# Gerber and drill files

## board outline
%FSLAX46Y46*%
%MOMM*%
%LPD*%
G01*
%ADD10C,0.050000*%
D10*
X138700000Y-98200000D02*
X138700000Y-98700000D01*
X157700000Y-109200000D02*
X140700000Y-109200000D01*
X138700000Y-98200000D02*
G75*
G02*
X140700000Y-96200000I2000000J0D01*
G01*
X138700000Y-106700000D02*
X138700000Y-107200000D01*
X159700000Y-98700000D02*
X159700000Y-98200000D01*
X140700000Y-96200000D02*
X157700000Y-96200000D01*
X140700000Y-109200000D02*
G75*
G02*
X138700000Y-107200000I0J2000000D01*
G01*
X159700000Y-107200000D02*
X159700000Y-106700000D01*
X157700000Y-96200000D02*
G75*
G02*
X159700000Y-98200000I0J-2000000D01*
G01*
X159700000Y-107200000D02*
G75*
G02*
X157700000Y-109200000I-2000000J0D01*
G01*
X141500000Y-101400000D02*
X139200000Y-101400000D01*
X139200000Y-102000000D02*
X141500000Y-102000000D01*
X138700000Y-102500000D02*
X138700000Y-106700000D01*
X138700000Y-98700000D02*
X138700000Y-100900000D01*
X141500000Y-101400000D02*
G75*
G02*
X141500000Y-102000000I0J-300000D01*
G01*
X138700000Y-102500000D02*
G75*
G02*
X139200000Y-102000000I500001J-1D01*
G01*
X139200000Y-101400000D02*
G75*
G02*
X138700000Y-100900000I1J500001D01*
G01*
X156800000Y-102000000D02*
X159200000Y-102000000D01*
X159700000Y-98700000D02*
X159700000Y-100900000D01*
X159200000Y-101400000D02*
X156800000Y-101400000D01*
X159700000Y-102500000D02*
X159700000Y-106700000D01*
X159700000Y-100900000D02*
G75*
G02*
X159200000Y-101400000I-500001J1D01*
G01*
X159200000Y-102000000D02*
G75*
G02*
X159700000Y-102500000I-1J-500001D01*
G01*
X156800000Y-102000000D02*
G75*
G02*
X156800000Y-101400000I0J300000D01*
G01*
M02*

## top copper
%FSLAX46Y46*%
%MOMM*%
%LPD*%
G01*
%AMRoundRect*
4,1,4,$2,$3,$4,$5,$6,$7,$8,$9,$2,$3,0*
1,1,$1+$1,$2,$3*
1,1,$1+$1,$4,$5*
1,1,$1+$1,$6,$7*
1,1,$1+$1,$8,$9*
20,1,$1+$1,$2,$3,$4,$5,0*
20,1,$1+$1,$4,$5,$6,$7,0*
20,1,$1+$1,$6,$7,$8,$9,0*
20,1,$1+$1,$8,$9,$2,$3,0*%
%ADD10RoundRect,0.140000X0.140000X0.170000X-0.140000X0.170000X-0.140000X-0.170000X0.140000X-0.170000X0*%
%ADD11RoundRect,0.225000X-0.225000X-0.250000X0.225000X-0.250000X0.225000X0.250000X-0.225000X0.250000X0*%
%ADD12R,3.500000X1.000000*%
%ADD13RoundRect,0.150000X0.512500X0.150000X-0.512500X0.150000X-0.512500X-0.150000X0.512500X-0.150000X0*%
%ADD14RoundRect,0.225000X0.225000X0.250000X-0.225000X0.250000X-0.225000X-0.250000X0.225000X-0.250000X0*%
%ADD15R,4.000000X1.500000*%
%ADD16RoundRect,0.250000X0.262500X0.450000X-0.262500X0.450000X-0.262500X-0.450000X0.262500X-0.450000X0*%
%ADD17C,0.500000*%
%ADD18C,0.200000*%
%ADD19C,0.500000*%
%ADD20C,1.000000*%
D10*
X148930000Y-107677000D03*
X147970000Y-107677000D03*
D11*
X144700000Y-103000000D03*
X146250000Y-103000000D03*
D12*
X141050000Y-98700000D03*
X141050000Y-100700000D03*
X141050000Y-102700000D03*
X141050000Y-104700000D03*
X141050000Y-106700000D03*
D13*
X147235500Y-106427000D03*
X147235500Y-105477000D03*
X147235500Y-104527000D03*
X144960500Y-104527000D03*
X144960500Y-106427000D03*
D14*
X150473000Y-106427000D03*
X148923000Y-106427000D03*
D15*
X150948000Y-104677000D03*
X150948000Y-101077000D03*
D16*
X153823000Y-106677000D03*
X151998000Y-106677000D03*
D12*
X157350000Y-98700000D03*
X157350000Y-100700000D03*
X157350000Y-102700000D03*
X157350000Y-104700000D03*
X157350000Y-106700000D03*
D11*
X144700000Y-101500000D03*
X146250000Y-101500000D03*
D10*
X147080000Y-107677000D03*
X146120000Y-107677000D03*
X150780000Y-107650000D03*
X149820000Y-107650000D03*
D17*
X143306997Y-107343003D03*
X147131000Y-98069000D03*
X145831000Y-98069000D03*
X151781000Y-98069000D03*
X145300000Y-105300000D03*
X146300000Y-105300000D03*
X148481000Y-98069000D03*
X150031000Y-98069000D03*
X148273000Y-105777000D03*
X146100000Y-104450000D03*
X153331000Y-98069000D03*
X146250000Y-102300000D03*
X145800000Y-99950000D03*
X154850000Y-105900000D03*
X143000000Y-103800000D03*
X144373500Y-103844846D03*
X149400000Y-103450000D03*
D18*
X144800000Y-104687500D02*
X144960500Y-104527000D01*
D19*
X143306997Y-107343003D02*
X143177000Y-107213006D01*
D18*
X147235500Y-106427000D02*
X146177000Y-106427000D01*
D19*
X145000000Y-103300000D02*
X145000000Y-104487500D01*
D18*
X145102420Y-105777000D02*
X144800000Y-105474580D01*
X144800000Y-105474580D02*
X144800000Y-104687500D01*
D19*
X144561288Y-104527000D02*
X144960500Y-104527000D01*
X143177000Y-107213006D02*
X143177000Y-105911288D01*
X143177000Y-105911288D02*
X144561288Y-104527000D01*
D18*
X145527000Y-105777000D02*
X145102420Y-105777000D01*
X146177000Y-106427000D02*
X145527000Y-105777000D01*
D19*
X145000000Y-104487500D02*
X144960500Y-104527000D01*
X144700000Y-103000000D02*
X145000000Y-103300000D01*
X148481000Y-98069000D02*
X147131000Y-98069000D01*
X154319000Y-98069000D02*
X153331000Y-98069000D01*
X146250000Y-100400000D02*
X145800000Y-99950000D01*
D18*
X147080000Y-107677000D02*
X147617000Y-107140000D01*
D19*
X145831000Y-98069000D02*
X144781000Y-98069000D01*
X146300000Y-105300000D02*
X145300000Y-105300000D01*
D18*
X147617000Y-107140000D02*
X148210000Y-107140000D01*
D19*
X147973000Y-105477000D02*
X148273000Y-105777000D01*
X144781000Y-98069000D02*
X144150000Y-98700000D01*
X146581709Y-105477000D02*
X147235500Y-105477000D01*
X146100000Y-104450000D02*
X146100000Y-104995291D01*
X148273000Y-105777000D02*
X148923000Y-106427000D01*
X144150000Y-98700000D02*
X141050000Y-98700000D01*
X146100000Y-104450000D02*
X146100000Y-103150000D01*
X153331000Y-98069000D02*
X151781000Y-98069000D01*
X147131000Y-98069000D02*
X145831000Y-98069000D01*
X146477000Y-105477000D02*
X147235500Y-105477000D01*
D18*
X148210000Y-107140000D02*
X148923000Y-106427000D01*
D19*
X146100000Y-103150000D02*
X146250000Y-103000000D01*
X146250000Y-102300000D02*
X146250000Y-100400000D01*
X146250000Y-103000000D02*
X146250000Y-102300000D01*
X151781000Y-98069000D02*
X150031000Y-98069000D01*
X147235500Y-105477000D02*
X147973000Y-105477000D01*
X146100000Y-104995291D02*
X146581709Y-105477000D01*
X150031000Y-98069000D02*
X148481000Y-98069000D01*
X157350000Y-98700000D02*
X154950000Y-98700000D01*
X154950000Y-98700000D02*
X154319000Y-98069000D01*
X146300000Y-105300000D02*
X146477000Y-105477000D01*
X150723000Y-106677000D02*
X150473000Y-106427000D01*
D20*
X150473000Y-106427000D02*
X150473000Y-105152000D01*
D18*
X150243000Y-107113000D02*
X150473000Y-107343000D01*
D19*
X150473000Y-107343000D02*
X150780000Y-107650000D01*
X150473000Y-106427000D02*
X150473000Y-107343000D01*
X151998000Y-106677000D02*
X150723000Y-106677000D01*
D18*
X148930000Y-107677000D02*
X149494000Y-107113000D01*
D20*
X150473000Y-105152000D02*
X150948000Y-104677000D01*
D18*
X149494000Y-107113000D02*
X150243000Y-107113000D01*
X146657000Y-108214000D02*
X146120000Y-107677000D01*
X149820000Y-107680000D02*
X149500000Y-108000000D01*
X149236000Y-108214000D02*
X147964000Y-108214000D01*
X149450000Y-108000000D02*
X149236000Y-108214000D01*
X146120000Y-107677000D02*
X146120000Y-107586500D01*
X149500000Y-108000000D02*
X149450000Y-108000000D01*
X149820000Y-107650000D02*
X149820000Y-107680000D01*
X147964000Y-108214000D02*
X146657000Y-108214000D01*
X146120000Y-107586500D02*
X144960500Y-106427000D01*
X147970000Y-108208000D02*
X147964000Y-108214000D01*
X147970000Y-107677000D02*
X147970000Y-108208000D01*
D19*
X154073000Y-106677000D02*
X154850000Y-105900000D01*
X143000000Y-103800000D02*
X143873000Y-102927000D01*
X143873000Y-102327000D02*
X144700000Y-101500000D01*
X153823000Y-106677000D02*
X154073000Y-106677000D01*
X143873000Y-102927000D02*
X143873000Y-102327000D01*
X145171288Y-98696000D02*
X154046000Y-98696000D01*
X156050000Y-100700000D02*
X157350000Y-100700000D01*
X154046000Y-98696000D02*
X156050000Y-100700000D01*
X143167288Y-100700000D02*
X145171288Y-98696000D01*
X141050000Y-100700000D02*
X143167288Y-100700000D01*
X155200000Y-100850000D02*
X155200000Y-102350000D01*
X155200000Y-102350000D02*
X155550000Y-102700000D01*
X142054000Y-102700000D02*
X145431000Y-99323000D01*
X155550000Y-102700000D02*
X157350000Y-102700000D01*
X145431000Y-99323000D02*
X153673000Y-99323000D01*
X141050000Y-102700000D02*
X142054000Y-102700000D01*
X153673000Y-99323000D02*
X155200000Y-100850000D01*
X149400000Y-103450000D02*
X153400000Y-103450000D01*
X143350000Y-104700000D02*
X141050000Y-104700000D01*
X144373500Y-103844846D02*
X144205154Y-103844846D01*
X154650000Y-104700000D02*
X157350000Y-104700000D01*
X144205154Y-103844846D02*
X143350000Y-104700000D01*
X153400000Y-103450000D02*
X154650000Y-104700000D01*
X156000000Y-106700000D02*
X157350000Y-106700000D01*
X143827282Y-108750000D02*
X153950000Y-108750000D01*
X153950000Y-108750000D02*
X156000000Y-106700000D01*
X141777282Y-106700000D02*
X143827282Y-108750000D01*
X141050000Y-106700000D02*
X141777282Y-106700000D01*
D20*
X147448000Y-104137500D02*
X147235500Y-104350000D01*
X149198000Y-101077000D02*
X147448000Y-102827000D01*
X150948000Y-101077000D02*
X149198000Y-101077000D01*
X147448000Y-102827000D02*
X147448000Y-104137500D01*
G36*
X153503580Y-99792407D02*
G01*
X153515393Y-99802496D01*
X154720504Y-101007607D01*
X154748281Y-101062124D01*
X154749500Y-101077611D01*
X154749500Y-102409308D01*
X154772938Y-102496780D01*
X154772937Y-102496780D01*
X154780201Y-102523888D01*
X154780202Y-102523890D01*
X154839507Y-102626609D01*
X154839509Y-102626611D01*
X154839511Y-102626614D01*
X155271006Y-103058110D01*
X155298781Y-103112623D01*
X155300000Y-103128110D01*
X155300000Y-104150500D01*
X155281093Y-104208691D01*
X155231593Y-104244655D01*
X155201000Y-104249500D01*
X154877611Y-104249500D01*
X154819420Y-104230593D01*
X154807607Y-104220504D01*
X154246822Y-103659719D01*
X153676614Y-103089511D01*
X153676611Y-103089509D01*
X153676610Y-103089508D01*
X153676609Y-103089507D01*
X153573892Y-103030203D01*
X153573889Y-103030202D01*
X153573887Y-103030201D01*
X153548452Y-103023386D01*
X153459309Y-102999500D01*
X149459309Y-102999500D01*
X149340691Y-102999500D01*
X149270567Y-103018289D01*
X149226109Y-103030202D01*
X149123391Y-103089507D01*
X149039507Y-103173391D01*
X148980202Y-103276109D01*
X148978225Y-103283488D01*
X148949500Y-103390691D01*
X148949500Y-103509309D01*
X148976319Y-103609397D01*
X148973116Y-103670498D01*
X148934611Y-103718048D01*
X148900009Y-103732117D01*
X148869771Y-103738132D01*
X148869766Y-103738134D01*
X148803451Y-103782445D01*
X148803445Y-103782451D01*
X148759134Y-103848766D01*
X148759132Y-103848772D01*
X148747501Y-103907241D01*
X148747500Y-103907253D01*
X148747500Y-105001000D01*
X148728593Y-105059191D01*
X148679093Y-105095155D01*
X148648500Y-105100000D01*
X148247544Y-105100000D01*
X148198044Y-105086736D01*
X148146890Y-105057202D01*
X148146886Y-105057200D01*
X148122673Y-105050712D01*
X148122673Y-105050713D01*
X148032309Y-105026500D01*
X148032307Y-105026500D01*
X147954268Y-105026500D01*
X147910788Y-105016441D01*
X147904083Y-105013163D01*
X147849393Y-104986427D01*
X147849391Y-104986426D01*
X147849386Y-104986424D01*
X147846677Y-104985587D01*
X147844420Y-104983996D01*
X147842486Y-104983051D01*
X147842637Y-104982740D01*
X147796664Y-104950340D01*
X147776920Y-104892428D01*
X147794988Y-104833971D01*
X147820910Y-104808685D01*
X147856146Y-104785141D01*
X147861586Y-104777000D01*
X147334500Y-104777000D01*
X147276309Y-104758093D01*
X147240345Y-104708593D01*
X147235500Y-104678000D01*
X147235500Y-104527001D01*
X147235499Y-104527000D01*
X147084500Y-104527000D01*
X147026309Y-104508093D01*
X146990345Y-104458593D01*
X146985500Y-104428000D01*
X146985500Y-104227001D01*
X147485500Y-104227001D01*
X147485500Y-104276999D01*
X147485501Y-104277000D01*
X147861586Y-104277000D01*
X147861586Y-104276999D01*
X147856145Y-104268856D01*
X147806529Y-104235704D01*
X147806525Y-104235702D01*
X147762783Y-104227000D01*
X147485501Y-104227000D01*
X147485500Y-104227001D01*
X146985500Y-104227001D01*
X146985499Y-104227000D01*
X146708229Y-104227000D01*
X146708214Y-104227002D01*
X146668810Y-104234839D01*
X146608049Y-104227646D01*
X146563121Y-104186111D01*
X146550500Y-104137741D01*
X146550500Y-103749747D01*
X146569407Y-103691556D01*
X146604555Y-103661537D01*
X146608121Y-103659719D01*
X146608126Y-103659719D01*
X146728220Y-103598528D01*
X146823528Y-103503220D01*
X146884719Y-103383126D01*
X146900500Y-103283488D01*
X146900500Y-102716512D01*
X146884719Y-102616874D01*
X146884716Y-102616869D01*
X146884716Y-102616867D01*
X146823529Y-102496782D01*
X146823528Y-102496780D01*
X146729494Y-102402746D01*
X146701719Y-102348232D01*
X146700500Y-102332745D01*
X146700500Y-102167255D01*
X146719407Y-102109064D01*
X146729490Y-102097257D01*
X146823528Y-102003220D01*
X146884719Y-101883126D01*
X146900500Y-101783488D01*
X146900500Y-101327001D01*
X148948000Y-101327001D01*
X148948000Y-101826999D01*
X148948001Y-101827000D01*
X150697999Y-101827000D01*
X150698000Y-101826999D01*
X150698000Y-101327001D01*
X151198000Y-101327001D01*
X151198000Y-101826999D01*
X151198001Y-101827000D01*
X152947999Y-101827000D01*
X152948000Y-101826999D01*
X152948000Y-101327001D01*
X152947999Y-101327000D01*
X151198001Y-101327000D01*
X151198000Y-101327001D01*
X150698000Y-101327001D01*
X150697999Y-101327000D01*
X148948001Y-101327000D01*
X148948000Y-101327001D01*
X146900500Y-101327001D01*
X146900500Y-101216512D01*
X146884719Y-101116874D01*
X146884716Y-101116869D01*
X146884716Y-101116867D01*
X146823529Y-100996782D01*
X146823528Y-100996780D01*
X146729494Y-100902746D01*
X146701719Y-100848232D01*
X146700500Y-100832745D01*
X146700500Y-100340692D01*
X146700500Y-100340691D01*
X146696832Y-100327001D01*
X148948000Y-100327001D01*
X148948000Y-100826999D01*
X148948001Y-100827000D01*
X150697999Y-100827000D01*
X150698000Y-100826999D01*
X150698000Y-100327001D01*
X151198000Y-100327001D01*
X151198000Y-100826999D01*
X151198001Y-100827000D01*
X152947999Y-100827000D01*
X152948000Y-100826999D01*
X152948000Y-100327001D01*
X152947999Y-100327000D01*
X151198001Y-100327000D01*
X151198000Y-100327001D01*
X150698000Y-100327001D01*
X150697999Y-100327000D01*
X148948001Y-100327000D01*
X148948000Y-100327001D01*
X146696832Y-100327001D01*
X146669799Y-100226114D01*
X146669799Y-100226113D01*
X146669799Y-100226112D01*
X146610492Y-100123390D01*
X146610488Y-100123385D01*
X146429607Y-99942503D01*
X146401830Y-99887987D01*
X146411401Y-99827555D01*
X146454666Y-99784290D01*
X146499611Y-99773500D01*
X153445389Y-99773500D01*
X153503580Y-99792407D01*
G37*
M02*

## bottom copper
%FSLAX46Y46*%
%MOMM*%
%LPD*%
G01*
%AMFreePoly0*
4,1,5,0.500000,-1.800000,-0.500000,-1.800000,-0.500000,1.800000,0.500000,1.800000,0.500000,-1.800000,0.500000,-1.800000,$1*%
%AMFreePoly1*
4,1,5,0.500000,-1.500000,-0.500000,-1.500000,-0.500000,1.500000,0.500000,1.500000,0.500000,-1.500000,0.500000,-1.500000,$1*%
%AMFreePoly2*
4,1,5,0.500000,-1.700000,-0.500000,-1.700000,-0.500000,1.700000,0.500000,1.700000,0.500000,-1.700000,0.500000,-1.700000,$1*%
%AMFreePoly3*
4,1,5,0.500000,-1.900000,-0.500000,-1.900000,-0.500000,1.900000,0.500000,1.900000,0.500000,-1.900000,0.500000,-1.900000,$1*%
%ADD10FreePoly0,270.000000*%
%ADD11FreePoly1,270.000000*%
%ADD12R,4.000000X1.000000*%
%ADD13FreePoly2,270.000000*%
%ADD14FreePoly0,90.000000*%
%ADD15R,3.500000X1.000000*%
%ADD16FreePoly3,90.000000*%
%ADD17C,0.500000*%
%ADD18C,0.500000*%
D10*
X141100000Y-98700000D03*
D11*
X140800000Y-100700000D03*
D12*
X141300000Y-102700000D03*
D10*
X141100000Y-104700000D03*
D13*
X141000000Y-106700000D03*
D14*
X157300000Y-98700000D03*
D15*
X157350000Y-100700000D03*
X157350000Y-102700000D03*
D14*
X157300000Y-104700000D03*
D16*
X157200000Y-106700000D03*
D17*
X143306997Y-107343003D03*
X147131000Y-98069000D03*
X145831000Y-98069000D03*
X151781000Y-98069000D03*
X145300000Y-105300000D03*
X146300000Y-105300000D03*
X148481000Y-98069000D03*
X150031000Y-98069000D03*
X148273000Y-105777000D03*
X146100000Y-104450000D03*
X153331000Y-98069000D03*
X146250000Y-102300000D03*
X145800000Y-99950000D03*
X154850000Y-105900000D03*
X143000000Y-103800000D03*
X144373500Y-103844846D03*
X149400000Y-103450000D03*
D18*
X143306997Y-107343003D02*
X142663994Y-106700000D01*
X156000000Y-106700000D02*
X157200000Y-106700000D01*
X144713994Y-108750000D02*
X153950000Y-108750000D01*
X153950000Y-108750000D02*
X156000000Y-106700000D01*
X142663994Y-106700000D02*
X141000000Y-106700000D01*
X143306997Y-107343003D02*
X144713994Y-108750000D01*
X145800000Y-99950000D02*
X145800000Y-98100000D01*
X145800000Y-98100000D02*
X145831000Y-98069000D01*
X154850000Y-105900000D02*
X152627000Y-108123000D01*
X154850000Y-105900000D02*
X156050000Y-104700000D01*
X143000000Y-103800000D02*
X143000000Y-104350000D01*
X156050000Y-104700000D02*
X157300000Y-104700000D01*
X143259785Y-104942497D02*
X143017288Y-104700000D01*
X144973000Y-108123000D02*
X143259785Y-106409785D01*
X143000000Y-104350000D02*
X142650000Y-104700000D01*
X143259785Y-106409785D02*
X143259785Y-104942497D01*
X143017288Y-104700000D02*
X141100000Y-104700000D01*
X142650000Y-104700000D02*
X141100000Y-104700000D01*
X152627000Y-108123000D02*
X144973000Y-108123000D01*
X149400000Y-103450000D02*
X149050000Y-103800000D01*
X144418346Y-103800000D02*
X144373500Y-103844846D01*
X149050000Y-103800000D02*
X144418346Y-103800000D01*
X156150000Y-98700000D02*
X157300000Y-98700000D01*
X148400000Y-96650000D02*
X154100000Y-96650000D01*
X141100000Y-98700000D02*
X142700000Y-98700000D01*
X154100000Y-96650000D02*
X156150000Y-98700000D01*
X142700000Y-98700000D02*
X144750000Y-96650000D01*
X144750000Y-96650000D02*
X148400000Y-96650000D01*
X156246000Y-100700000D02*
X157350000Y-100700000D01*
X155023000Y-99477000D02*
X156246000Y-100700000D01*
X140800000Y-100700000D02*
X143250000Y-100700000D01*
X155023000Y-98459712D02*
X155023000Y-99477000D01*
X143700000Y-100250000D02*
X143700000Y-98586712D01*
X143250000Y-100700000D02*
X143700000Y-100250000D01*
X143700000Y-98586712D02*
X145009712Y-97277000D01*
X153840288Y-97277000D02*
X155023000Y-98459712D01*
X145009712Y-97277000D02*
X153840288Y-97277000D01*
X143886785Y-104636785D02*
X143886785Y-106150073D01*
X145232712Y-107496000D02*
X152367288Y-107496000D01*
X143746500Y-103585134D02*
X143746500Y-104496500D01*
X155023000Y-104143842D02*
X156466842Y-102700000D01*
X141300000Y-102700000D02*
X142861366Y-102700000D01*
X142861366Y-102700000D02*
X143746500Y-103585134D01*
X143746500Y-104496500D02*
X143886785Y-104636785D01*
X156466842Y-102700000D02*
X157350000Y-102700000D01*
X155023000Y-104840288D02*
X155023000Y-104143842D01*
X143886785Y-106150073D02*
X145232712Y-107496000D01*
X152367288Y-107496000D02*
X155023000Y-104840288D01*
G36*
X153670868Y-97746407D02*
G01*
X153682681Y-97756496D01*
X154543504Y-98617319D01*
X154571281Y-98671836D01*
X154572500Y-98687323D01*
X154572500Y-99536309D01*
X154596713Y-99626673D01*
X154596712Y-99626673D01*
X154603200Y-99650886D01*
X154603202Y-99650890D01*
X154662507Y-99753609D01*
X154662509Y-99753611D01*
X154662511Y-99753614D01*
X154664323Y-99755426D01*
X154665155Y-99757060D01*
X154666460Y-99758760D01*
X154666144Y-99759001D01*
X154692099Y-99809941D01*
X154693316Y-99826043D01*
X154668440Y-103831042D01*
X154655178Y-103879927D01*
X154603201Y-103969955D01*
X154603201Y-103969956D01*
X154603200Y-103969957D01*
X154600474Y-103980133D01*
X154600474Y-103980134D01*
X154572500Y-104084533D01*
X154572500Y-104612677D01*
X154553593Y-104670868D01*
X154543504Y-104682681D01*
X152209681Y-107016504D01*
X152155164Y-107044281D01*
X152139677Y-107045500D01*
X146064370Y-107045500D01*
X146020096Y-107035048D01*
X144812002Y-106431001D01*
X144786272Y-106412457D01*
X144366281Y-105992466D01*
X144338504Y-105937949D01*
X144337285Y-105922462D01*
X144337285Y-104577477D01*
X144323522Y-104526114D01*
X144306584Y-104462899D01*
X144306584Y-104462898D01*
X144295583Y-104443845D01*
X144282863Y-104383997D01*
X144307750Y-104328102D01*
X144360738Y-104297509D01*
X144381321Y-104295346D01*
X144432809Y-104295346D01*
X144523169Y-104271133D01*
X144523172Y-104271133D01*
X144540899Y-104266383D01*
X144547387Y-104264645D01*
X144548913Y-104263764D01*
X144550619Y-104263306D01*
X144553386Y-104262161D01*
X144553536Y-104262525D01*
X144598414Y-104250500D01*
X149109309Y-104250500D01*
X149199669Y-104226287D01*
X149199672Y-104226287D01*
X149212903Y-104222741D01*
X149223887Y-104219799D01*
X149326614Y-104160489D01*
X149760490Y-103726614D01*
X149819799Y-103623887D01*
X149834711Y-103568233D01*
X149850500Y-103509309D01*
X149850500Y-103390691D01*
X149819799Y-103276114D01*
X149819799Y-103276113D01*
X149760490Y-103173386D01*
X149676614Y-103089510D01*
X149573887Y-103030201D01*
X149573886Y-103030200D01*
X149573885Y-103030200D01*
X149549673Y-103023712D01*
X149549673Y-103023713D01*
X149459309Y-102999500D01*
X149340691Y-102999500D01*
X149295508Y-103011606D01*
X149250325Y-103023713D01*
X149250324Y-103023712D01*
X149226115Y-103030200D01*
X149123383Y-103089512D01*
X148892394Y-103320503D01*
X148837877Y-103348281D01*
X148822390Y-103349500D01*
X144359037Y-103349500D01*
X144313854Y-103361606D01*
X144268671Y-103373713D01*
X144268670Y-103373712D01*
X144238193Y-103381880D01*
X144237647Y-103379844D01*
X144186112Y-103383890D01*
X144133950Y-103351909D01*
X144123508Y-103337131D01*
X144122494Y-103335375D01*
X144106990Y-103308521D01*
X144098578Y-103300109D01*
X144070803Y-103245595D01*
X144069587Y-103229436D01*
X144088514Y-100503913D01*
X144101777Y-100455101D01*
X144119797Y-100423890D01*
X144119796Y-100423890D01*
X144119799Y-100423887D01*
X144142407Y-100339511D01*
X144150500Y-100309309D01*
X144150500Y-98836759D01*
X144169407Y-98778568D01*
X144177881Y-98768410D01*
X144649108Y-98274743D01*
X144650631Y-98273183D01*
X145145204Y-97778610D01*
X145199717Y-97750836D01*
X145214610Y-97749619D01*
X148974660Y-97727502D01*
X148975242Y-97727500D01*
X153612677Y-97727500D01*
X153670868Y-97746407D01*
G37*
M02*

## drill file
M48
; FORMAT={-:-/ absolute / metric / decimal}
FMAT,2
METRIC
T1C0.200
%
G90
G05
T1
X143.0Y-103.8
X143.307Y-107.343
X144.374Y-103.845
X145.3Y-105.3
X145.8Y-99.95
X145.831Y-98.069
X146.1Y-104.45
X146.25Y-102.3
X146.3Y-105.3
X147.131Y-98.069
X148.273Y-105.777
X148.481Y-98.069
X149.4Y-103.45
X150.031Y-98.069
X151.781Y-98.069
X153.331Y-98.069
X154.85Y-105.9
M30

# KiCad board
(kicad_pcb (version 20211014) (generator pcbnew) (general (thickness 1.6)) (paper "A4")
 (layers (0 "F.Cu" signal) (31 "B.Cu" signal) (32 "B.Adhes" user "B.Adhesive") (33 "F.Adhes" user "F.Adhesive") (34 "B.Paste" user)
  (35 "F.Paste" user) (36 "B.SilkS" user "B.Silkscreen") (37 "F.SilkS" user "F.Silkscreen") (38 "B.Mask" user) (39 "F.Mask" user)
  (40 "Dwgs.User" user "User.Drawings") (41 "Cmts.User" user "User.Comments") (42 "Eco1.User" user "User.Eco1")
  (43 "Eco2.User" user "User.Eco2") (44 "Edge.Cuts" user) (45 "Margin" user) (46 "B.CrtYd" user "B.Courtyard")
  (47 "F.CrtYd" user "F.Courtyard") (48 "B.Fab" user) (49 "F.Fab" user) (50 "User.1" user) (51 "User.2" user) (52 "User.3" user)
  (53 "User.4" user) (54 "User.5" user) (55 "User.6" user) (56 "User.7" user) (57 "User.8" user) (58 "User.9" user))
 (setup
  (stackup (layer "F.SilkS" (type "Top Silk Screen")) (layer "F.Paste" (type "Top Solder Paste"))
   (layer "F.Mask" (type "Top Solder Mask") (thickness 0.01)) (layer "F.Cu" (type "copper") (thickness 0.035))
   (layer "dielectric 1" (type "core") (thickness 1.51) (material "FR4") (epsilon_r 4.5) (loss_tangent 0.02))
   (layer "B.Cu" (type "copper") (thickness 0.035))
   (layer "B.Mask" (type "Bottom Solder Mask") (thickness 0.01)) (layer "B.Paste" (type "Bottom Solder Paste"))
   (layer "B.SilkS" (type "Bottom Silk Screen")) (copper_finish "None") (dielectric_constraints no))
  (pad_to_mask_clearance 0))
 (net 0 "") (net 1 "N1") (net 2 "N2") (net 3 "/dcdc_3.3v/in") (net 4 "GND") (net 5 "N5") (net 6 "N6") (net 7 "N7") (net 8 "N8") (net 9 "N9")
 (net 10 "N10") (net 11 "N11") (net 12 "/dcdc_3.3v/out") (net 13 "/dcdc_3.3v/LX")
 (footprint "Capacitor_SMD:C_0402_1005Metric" (layer "F.Cu") (at 148.45 107.677 180)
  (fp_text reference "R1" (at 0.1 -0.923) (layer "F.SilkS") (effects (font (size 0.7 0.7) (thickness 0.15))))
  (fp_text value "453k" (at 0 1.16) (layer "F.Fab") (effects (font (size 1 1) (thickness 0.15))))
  (pad "1" smd roundrect (at -0.48 0 180) (size 0.56 0.62) (layers "F.Cu" "F.Paste" "F.Mask") (roundrect_rratio 0.25) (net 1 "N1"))
  (pad "2" smd roundrect (at 0.48 0 180) (size 0.56 0.62) (layers "F.Cu" "F.Paste" "F.Mask") (roundrect_rratio 0.25) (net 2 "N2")))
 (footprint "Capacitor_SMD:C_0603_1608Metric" (layer "F.Cu") (at 145.475 103)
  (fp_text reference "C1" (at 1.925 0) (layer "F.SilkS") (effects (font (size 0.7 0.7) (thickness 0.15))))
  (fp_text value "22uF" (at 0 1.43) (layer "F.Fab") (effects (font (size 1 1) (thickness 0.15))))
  (pad "1" smd roundrect (at -0.775 0) (size 0.9 0.95) (layers "F.Cu" "F.Paste" "F.Mask") (roundrect_rratio 0.25) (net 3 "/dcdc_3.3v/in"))
  (pad "2" smd roundrect (at 0.775 0) (size 0.9 0.95) (layers "F.Cu" "F.Paste" "F.Mask") (roundrect_rratio 0.25) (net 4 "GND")))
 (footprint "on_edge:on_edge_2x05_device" (layer "F.Cu") (at 138.7 102.7 -90)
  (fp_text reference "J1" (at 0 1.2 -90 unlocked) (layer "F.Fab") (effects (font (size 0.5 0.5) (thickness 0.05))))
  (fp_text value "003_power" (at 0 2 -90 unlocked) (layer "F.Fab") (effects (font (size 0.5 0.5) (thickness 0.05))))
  (fp_line (start -1.3 -2.8) (end -1.3 -0.5) (layer "Edge.Cuts") (width 0.05))
  (fp_line (start -0.7 -0.5) (end -0.7 -2.8) (layer "Edge.Cuts") (width 0.05))
  (fp_line (start -0.2 0) (end 4 0) (layer "Edge.Cuts") (width 0.05))
  (fp_line (start -4 0) (end -1.8 0) (layer "Edge.Cuts") (width 0.05))
  (fp_arc (start -1.3 -2.8) (mid -1 -3.1) (end -0.7 -2.8) (layer "Edge.Cuts") (width 0.05))
  (fp_arc (start -0.2 0) (mid -0.553553 -0.146447) (end -0.7 -0.5) (layer "Edge.Cuts") (width 0.05))
  (fp_arc (start -1.3 -0.5) (mid -1.446447 -0.146447) (end -1.8 0) (layer "Edge.Cuts") (width 0.05))
  (pad "1" smd rect (at -4 -2.35 90) (size 1 3.5) (layers "F.Cu" "F.Mask") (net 4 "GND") (zone_connect 0))
  (pad "2" smd rect (at -2 -2.35 270) (size 1 3.5) (layers "F.Cu" "F.Mask") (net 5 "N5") (zone_connect 0))
  (pad "3" smd rect (at 0 -2.35 270) (size 1 3.5) (layers "F.Cu" "F.Mask") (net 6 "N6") (zone_connect 0))
  (pad "4" smd rect (at 2 -2.35 90) (size 1 3.5) (layers "F.Cu" "F.Mask") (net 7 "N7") (zone_connect 0))
  (pad "5" smd rect (at 4 -2.35 90) (size 1 3.5) (layers "F.Cu" "F.Mask") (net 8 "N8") (zone_connect 0))
  (pad "6" smd custom (at -4 -2.4 270) (size 1 3.6) (layers "B.Cu" "B.Mask") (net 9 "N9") (zone_connect 0)
   (options (clearance outline) (anchor rect)) (primitives))
  (pad "7" smd custom (at -2 -2.1 270) (size 1 3) (layers "B.Cu" "B.Mask") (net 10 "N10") (zone_connect 0)
   (options (clearance outline) (anchor rect)) (primitives))
  (pad "8" smd rect (at 0 -2.6 270) (size 1 4) (layers "B.Cu" "B.Mask") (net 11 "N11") (zone_connect 0))
  (pad "9" smd custom (at 2 -2.4 270) (size 1 3.6) (layers "B.Cu" "B.Mask") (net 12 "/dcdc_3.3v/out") (zone_connect 0)
   (options (clearance outline) (anchor rect)) (primitives))
  (pad "10" smd custom (at 4 -2.3 270) (size 1 3.4) (layers "B.Cu" "B.Mask") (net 3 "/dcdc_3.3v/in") (zone_connect 0)
   (options (clearance outline) (anchor rect)) (primitives))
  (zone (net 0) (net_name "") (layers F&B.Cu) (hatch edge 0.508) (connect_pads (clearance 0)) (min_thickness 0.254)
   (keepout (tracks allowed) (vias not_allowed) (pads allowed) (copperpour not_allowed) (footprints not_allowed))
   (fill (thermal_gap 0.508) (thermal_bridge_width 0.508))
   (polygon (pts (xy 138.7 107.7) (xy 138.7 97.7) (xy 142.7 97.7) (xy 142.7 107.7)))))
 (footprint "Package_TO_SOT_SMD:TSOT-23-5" (layer "F.Cu") (at 146.098 105.477 180)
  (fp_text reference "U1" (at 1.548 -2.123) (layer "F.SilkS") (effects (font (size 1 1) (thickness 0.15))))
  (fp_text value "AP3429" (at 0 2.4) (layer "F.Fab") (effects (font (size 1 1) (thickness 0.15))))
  (pad "1" smd roundrect (at -1.1375 -0.95 180) (size 1.325 0.6) (layers "F.Cu" "F.Paste" "F.Mask") (roundrect_rratio 0.25)
   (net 3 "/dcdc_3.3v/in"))
  (pad "2" smd roundrect (at -1.1375 0 180) (size 1.325 0.6) (layers "F.Cu" "F.Paste" "F.Mask") (roundrect_rratio 0.25) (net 4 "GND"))
  (pad "3" smd roundrect (at -1.1375 0.95 180) (size 1.325 0.6) (layers "F.Cu" "F.Paste" "F.Mask") (roundrect_rratio 0.25)
   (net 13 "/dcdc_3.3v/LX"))
  (pad "4" smd roundrect (at 1.1375 0.95 180) (size 1.325 0.6) (layers "F.Cu" "F.Paste" "F.Mask") (roundrect_rratio 0.25)
   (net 3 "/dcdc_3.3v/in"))
  (pad "5" smd roundrect (at 1.1375 -0.95 180) (size 1.325 0.6) (layers "F.Cu" "F.Paste" "F.Mask") (roundrect_rratio 0.25) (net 2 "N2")))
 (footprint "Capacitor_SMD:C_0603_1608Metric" (layer "F.Cu") (at 149.698 106.427 180)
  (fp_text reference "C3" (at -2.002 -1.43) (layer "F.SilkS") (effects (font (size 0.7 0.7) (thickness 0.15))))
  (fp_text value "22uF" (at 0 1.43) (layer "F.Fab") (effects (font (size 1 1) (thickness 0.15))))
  (pad "1" smd roundrect (at -0.775 0 180) (size 0.9 0.95) (layers "F.Cu" "F.Paste" "F.Mask") (roundrect_rratio 0.25) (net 1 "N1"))
  (pad "2" smd roundrect (at 0.775 0 180) (size 0.9 0.95) (layers "F.Cu" "F.Paste" "F.Mask") (roundrect_rratio 0.25) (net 4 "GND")))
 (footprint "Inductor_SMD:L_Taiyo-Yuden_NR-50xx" (layer "F.Cu") (at 150.948 102.877 90)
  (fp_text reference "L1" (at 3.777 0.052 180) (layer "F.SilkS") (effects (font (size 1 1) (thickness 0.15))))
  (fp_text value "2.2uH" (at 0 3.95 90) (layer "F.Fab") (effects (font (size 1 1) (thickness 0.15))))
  (pad "1" smd rect (at -1.8 0 90) (size 1.5 4) (layers "F.Cu" "F.Paste" "F.Mask") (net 1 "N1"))
  (pad "2" smd rect (at 1.8 0 90) (size 1.5 4) (layers "F.Cu" "F.Paste" "F.Mask") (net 13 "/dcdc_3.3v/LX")))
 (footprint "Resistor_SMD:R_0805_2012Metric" (layer "F.Cu") (at 152.9105 106.677 180)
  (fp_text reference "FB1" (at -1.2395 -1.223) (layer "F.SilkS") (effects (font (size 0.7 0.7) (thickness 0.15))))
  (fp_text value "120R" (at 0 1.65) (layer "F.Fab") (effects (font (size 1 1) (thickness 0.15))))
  (pad "1" smd roundrect (at -0.9125 0 180) (size 1.025 1.4) (layers "F.Cu" "F.Paste" "F.Mask") (roundrect_rratio 0.243902)
   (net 12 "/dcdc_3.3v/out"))
  (pad "2" smd roundrect (at 0.9125 0 180) (size 1.025 1.4) (layers "F.Cu" "F.Paste" "F.Mask") (roundrect_rratio 0.243902) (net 1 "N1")))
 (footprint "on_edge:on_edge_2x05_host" (layer "F.Cu") (at 159.7 102.7 -90)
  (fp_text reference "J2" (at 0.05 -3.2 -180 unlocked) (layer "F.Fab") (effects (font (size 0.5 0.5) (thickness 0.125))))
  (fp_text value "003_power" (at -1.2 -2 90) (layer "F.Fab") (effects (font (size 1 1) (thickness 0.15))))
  (fp_line (start -0.7 2.9) (end -0.7 0.5) (layer "Edge.Cuts") (width 0.05))
  (fp_line (start -4 0) (end -1.8 0) (layer "Edge.Cuts") (width 0.05))
  (fp_line (start -1.3 0.5) (end -1.3 2.9) (layer "Edge.Cuts") (width 0.05))
  (fp_line (start -0.2 0) (end 4 0) (layer "Edge.Cuts") (width 0.05))
  (fp_arc (start -1.8 0) (mid -1.446447 0.146447) (end -1.3 0.5) (layer "Edge.Cuts") (width 0.05))
  (fp_arc (start -0.7 0.5) (mid -0.553553 0.146447) (end -0.2 0) (layer "Edge.Cuts") (width 0.05))
  (fp_arc (start -0.7 2.9) (mid -1 3.2) (end -1.3 2.9) (layer "Edge.Cuts") (width 0.05))
  (pad "1" smd rect (at -4 2.35 270) (size 1 3.5) (layers "F.Cu" "F.Mask") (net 4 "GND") (zone_connect 0))
  (pad "2" smd rect (at -2 2.35 270) (size 1 3.5) (layers "F.Cu" "F.Mask") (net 5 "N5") (zone_connect 0))
  (pad "3" smd rect (at 0 2.35 270) (size 1 3.5) (layers "F.Cu" "F.Mask") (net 6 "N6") (zone_connect 0))
  (pad "4" smd rect (at 2 2.35 270) (size 1 3.5) (layers "F.Cu" "F.Mask") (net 7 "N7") (zone_connect 0))
  (pad "5" smd rect (at 4 2.35 270) (size 1 3.5) (layers "F.Cu" "F.Mask") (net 8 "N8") (zone_connect 0))
  (pad "6" smd custom (at -4 2.4 90) (size 1 3.6) (layers "B.Cu" "B.Mask") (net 9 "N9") (zone_connect 0)
   (options (clearance outline) (anchor rect)) (primitives))
  (pad "7" smd rect (at -2 2.35 90) (size 1 3.5) (layers "B.Cu" "B.Mask") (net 10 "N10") (zone_connect 0))
  (pad "8" smd rect (at 0 2.35 90) (size 1 3.5) (layers "B.Cu" "B.Mask") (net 11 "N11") (zone_connect 0))
  (pad "9" smd custom (at 2 2.4 90) (size 1 3.6) (layers "B.Cu" "B.Mask") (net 12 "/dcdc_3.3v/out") (zone_connect 0)
   (options (clearance outline) (anchor rect)) (primitives))
  (pad "10" smd custom (at 4 2.5 90) (size 1 3.8) (layers "B.Cu" "B.Mask") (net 3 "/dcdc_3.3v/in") (zone_connect 0)
   (options (clearance outline) (anchor rect)) (primitives))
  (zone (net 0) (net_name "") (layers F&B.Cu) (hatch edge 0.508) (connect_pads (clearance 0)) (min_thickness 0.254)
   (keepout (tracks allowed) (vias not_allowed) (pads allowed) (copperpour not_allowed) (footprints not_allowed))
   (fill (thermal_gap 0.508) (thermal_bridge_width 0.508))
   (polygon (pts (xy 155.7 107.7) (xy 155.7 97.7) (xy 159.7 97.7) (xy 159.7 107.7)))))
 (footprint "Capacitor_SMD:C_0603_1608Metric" (layer "F.Cu") (at 145.475 101.5)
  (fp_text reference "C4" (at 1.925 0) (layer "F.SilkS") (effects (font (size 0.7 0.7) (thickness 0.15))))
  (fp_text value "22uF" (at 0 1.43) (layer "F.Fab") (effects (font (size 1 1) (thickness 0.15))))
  (pad "1" smd roundrect (at -0.775 0) (size 0.9 0.95) (layers "F.Cu" "F.Paste" "F.Mask") (roundrect_rratio 0.25) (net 12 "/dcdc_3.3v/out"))
  (pad "2" smd roundrect (at 0.775 0) (size 0.9 0.95) (layers "F.Cu" "F.Paste" "F.Mask") (roundrect_rratio 0.25) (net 4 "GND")))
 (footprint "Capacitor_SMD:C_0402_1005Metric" (layer "F.Cu") (at 146.6 107.677 180)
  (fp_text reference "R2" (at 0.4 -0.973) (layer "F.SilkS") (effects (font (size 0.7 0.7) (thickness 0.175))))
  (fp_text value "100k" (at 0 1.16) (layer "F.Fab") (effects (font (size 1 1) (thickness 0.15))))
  (pad "1" smd roundrect (at -0.48 0 180) (size 0.56 0.62) (layers "F.Cu" "F.Paste" "F.Mask") (roundrect_rratio 0.25) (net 4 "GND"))
  (pad "2" smd roundrect (at 0.48 0 180) (size 0.56 0.62) (layers "F.Cu" "F.Paste" "F.Mask") (roundrect_rratio 0.25) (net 2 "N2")))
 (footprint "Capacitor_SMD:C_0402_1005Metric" (layer "F.Cu") (at 150.3 107.65 180)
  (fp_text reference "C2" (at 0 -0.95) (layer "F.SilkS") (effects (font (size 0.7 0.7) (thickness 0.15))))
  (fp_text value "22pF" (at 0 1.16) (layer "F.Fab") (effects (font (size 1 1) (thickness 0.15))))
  (pad "1" smd roundrect (at -0.48 0 180) (size 0.56 0.62) (layers "F.Cu" "F.Paste" "F.Mask") (roundrect_rratio 0.25) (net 1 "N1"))
  (pad "2" smd roundrect (at 0.48 0 180) (size 0.56 0.62) (layers "F.Cu" "F.Paste" "F.Mask") (roundrect_rratio 0.25) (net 2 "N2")))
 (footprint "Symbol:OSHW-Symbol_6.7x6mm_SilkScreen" (layer "B.Cu") (at 148.95 102.7 180)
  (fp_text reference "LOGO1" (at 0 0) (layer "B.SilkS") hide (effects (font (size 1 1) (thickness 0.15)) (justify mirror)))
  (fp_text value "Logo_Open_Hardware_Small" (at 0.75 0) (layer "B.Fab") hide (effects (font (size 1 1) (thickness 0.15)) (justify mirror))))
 (gr_line (start 138.7 98.2) (end 138.7 98.7) (layer "Edge.Cuts") (width 0.05))
 (gr_line (start 157.7 109.2) (end 140.7 109.2) (layer "Edge.Cuts") (width 0.05))
 (gr_arc (start 138.7 98.2) (mid 139.285786 96.785786) (end 140.7 96.2) (layer "Edge.Cuts") (width 0.05))
 (gr_line (start 138.7 106.7) (end 138.7 107.2) (layer "Edge.Cuts") (width 0.05))
 (gr_line (start 159.7 98.7) (end 159.7 98.2) (layer "Edge.Cuts") (width 0.05))
 (gr_line (start 140.7 96.2) (end 157.7 96.2) (layer "Edge.Cuts") (width 0.05))
 (gr_arc (start 140.7 109.2) (mid 139.285786 108.614214) (end 138.7 107.2) (layer "Edge.Cuts") (width 0.05))
 (gr_line (start 159.7 107.2) (end 159.7 106.7) (layer "Edge.Cuts") (width 0.05))
 (gr_arc (start 157.7 96.2) (mid 159.114214 96.785786) (end 159.7 98.2) (layer "Edge.Cuts") (width 0.05))
 (gr_arc (start 159.7 107.2) (mid 159.114214 108.614214) (end 157.7 109.2) (layer "Edge.Cuts") (width 0.05))
 (segment (start 144.8 104.6875) (end 144.9605 104.527) (width 0.2) (layer "F.Cu") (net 3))
 (segment (start 143.306997 107.343003) (end 143.177 107.213006) (width 0.5) (layer "F.Cu") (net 3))
 (segment (start 147.2355 106.427) (end 146.177 106.427) (width 0.2) (layer "F.Cu") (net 3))
 (segment (start 145 103.3) (end 145 104.4875) (width 0.5) (layer "F.Cu") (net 3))
 (segment (start 145.10242 105.777) (end 144.8 105.47458) (width 0.2) (layer "F.Cu") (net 3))
 (segment (start 144.8 105.47458) (end 144.8 104.6875) (width 0.2) (layer "F.Cu") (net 3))
 (segment (start 144.561288 104.527) (end 144.9605 104.527) (width 0.5) (layer "F.Cu") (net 3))
 (segment (start 143.177 107.213006) (end 143.177 105.911288) (width 0.5) (layer "F.Cu") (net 3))
 (segment (start 143.177 105.911288) (end 144.561288 104.527) (width 0.5) (layer "F.Cu") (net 3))
 (segment (start 145.527 105.777) (end 145.10242 105.777) (width 0.2) (layer "F.Cu") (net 3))
 (segment (start 146.177 106.427) (end 145.527 105.777) (width 0.2) (layer "F.Cu") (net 3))
 (segment (start 145 104.4875) (end 144.9605 104.527) (width 0.5) (layer "F.Cu") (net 3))
 (segment (start 144.7 103) (end 145 103.3) (width 0.5) (layer "F.Cu") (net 3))
 (via (at 143.306997 107.343003) (size 0.5) (drill 0.2) (layers "F.Cu" "B.Cu") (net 3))
 (segment (start 143.306997 107.343003) (end 142.663994 106.7) (width 0.5) (layer "B.Cu") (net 3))
 (segment (start 156 106.7) (end 157.2 106.7) (width 0.5) (layer "B.Cu") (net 3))
 (segment (start 144.713994 108.75) (end 153.95 108.75) (width 0.5) (layer "B.Cu") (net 3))
 (segment (start 153.95 108.75) (end 156 106.7) (width 0.5) (layer "B.Cu") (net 3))
 (segment (start 142.663994 106.7) (end 141 106.7) (width 0.5) (layer "B.Cu") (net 3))
 (segment (start 143.306997 107.343003) (end 144.713994 108.75) (width 0.5) (layer "B.Cu") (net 3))
 (segment (start 148.481 98.069) (end 147.131 98.069) (width 0.5) (layer "F.Cu") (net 4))
 (segment (start 154.319 98.069) (end 153.331 98.069) (width 0.5) (layer "F.Cu") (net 4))
 (segment (start 146.25 100.4) (end 145.8 99.95) (width 0.5) (layer "F.Cu") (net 4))
 (segment (start 147.08 107.677) (end 147.617 107.14) (width 0.2) (layer "F.Cu") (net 4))
 (segment (start 145.831 98.069) (end 144.781 98.069) (width 0.5) (layer "F.Cu") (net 4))
 (segment (start 146.3 105.3) (end 145.3 105.3) (width 0.5) (layer "F.Cu") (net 4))
 (segment (start 147.617 107.14) (end 148.21 107.14) (width 0.2) (layer "F.Cu") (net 4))
 (segment (start 147.973 105.477) (end 148.273 105.777) (width 0.5) (layer "F.Cu") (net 4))
 (segment (start 144.781 98.069) (end 144.15 98.7) (width 0.5) (layer "F.Cu") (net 4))
 (segment (start 146.581709 105.477) (end 147.2355 105.477) (width 0.5) (layer "F.Cu") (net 4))
 (segment (start 146.1 104.45) (end 146.1 104.995291) (width 0.5) (layer "F.Cu") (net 4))
 (segment (start 148.273 105.777) (end 148.923 106.427) (width 0.5) (layer "F.Cu") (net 4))
 (segment (start 144.15 98.7) (end 141.05 98.7) (width 0.5) (layer "F.Cu") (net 4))
 (segment (start 146.1 104.45) (end 146.1 103.15) (width 0.5) (layer "F.Cu") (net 4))
 (segment (start 153.331 98.069) (end 151.781 98.069) (width 0.5) (layer "F.Cu") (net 4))
 (segment (start 147.131 98.069) (end 145.831 98.069) (width 0.5) (layer "F.Cu") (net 4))
 (segment (start 146.477 105.477) (end 147.2355 105.477) (width 0.5) (layer "F.Cu") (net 4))
 (segment (start 148.21 107.14) (end 148.923 106.427) (width 0.2) (layer "F.Cu") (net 4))
 (segment (start 146.1 103.15) (end 146.25 103) (width 0.5) (layer "F.Cu") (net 4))
 (segment (start 146.25 102.3) (end 146.25 100.4) (width 0.5) (layer "F.Cu") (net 4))
 (segment (start 146.25 103) (end 146.25 102.3) (width 0.5) (layer "F.Cu") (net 4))
 (segment (start 151.781 98.069) (end 150.031 98.069) (width 0.5) (layer "F.Cu") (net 4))
 (segment (start 147.2355 105.477) (end 147.973 105.477) (width 0.5) (layer "F.Cu") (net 4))
 (segment (start 146.1 104.995291) (end 146.581709 105.477) (width 0.5) (layer "F.Cu") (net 4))
 (segment (start 150.031 98.069) (end 148.481 98.069) (width 0.5) (layer "F.Cu") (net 4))
 (segment (start 157.35 98.7) (end 154.95 98.7) (width 0.5) (layer "F.Cu") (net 4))
 (segment (start 154.95 98.7) (end 154.319 98.069) (width 0.5) (layer "F.Cu") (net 4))
 (segment (start 146.3 105.3) (end 146.477 105.477) (width 0.5) (layer "F.Cu") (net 4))
 (via (at 147.131 98.069) (size 0.5) (drill 0.2) (layers "F.Cu" "B.Cu") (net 4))
 (via (at 145.831 98.069) (size 0.5) (drill 0.2) (layers "F.Cu" "B.Cu") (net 4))
 (via (at 151.781 98.069) (size 0.5) (drill 0.2) (layers "F.Cu" "B.Cu") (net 4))
 (via (at 145.3 105.3) (size 0.5) (drill 0.2) (layers "F.Cu" "B.Cu") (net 4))
 (via (at 146.3 105.3) (size 0.5) (drill 0.2) (layers "F.Cu" "B.Cu") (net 4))
 (via (at 148.481 98.069) (size 0.5) (drill 0.2) (layers "F.Cu" "B.Cu") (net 4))
 (via (at 150.031 98.069) (size 0.5) (drill 0.2) (layers "F.Cu" "B.Cu") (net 4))
 (via (at 148.273 105.777) (size 0.5) (drill 0.2) (layers "F.Cu" "B.Cu") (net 4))
 (via (at 146.1 104.45) (size 0.5) (drill 0.2) (layers "F.Cu" "B.Cu") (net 4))
 (via (at 153.331 98.069) (size 0.5) (drill 0.2) (layers "F.Cu" "B.Cu") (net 4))
 (via (at 146.25 102.3) (size 0.5) (drill 0.2) (layers "F.Cu" "B.Cu") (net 4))
 (via (at 145.8 99.95) (size 0.5) (drill 0.2) (layers "F.Cu" "B.Cu") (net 4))
 (segment (start 145.8 99.95) (end 145.8 98.1) (width 0.5) (layer "B.Cu") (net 4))
 (segment (start 145.8 98.1) (end 145.831 98.069) (width 0.5) (layer "B.Cu") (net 4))
 (segment (start 150.723 106.677) (end 150.473 106.427) (width 0.5) (layer "F.Cu") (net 1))
 (segment (start 150.473 106.427) (end 150.473 105.152) (width 1) (layer "F.Cu") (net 1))
 (segment (start 150.243 107.113) (end 150.473 107.343) (width 0.2) (layer "F.Cu") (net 1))
 (segment (start 150.473 107.343) (end 150.78 107.65) (width 0.5) (layer "F.Cu") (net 1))
 (segment (start 150.473 106.427) (end 150.473 107.343) (width 0.5) (layer "F.Cu") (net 1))
 (segment (start 151.998 106.677) (end 150.723 106.677) (width 0.5) (layer "F.Cu") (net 1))
 (segment (start 148.93 107.677) (end 149.494 107.113) (width 0.2) (layer "F.Cu") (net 1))
 (segment (start 150.473 105.152) (end 150.948 104.677) (width 1) (layer "F.Cu") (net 1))
 (segment (start 149.494 107.113) (end 150.243 107.113) (width 0.2) (layer "F.Cu") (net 1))
 (segment (start 146.657 108.214) (end 146.12 107.677) (width 0.2) (layer "F.Cu") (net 2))
 (segment (start 149.82 107.68) (end 149.5 108) (width 0.2) (layer "F.Cu") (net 2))
 (segment (start 149.236 108.214) (end 147.964 108.214) (width 0.2) (layer "F.Cu") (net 2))
 (segment (start 149.45 108) (end 149.236 108.214) (width 0.2) (layer "F.Cu") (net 2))
 (segment (start 146.12 107.677) (end 146.12 107.5865) (width 0.2) (layer "F.Cu") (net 2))
 (segment (start 149.5 108) (end 149.45 108) (width 0.2) (layer "F.Cu") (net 2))
 (segment (start 149.82 107.65) (end 149.82 107.68) (width 0.2) (layer "F.Cu") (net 2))
 (segment (start 147.964 108.214) (end 146.657 108.214) (width 0.2) (layer "F.Cu") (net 2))
 (segment (start 146.12 107.5865) (end 144.9605 106.427) (width 0.2) (layer "F.Cu") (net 2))
 (segment (start 147.97 108.208) (end 147.964 108.214) (width 0.2) (layer "F.Cu") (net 2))
 (segment (start 147.97 107.677) (end 147.97 108.208) (width 0.2) (layer "F.Cu") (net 2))
 (segment (start 154.073 106.677) (end 154.85 105.9) (width 0.5) (layer "F.Cu") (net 12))
 (segment (start 143 103.8) (end 143.873 102.927) (width 0.5) (layer "F.Cu") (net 12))
 (segment (start 143.873 102.327) (end 144.7 101.5) (width 0.5) (layer "F.Cu") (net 12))
 (segment (start 153.823 106.677) (end 154.073 106.677) (width 0.5) (layer "F.Cu") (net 12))
 (segment (start 143.873 102.927) (end 143.873 102.327) (width 0.5) (layer "F.Cu") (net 12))
 (via (at 154.85 105.9) (size 0.5) (drill 0.2) (layers "F.Cu" "B.Cu") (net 12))
 (via (at 143 103.8) (size 0.5) (drill 0.2) (layers "F.Cu" "B.Cu") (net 12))
 (segment (start 154.85 105.9) (end 152.627 108.123) (width 0.5) (layer "B.Cu") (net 12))
 (segment (start 154.85 105.9) (end 156.05 104.7) (width 0.5) (layer "B.Cu") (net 12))
 (segment (start 143 103.8) (end 143 104.35) (width 0.5) (layer "B.Cu") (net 12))
 (segment (start 156.05 104.7) (end 157.3 104.7) (width 0.5) (layer "B.Cu") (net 12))
 (segment (start 143.259785 104.942497) (end 143.017288 104.7) (width 0.5) (layer "B.Cu") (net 12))
 (segment (start 144.973 108.123) (end 143.259785 106.409785) (width 0.5) (layer "B.Cu") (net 12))
 (segment (start 143 104.35) (end 142.65 104.7) (width 0.5) (layer "B.Cu") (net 12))
 (segment (start 143.259785 106.409785) (end 143.259785 104.942497) (width 0.5) (layer "B.Cu") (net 12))
 (segment (start 143.017288 104.7) (end 141.1 104.7) (width 0.5) (layer "B.Cu") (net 12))
 (segment (start 142.65 104.7) (end 141.1 104.7) (width 0.5) (layer "B.Cu") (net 12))
 (segment (start 152.627 108.123) (end 144.973 108.123) (width 0.5) (layer "B.Cu") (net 12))
 (segment (start 145.171288 98.696) (end 154.046 98.696) (width 0.5) (layer "F.Cu") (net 5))
 (segment (start 156.05 100.7) (end 157.35 100.7) (width 0.5) (layer "F.Cu") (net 5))
 (segment (start 154.046 98.696) (end 156.05 100.7) (width 0.5) (layer "F.Cu") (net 5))
 (segment (start 143.167288 100.7) (end 145.171288 98.696) (width 0.5) (layer "F.Cu") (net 5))
 (segment (start 141.05 100.7) (end 143.167288 100.7) (width 0.5) (layer "F.Cu") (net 5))
 (segment (start 155.2 100.85) (end 155.2 102.35) (width 0.5) (layer "F.Cu") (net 6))
 (segment (start 155.2 102.35) (end 155.55 102.7) (width 0.5) (layer "F.Cu") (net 6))
 (segment (start 142.054 102.7) (end 145.431 99.323) (width 0.5) (layer "F.Cu") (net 6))
 (segment (start 155.55 102.7) (end 157.35 102.7) (width 0.5) (layer "F.Cu") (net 6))
 (segment (start 145.431 99.323) (end 153.673 99.323) (width 0.5) (layer "F.Cu") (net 6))
 (segment (start 141.05 102.7) (end 142.054 102.7) (width 0.5) (layer "F.Cu") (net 6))
 (segment (start 153.673 99.323) (end 155.2 100.85) (width 0.5) (layer "F.Cu") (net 6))
 (segment (start 149.4 103.45) (end 153.4 103.45) (width 0.5) (layer "F.Cu") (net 7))
 (segment (start 143.35 104.7) (end 141.05 104.7) (width 0.5) (layer "F.Cu") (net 7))
 (segment (start 144.3735 103.844846) (end 144.205154 103.844846) (width 0.5) (layer "F.Cu") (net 7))
 (segment (start 154.65 104.7) (end 157.35 104.7) (width 0.5) (layer "F.Cu") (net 7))
 (segment (start 144.205154 103.844846) (end 143.35 104.7) (width 0.5) (layer "F.Cu") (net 7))
 (segment (start 153.4 103.45) (end 154.65 104.7) (width 0.5) (layer "F.Cu") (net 7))
 (via (at 144.3735 103.844846) (size 0.5) (drill 0.2) (layers "F.Cu" "B.Cu") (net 7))
 (via (at 149.4 103.45) (size 0.5) (drill 0.2) (layers "F.Cu" "B.Cu") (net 7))
 (segment (start 149.4 103.45) (end 149.05 103.8) (width 0.5) (layer "B.Cu") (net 7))
 (segment (start 144.418346 103.8) (end 144.3735 103.844846) (width 0.5) (layer "B.Cu") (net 7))
 (segment (start 149.05 103.8) (end 144.418346 103.8) (width 0.5) (layer "B.Cu") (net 7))
 (segment (start 156 106.7) (end 157.35 106.7) (width 0.5) (layer "F.Cu") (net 8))
 (segment (start 143.827282 108.75) (end 153.95 108.75) (width 0.5) (layer "F.Cu") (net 8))
 (segment (start 153.95 108.75) (end 156 106.7) (width 0.5) (layer "F.Cu") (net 8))
 (segment (start 141.777282 106.7) (end 143.827282 108.75) (width 0.5) (layer "F.Cu") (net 8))
 (segment (start 141.05 106.7) (end 141.777282 106.7) (width 0.5) (layer "F.Cu") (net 8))
 (segment (start 156.15 98.7) (end 157.3 98.7) (width 0.5) (layer "B.Cu") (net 9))
 (segment (start 148.4 96.65) (end 154.1 96.65) (width 0.5) (layer "B.Cu") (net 9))
 (segment (start 141.1 98.7) (end 142.7 98.7) (width 0.5) (layer "B.Cu") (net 9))
 (segment (start 154.1 96.65) (end 156.15 98.7) (width 0.5) (layer "B.Cu") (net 9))
 (segment (start 142.7 98.7) (end 144.75 96.65) (width 0.5) (layer "B.Cu") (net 9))
 (segment (start 144.75 96.65) (end 148.4 96.65) (width 0.5) (layer "B.Cu") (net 9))
 (segment (start 156.246 100.7) (end 157.35 100.7) (width 0.5) (layer "B.Cu") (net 10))
 (segment (start 155.023 99.477) (end 156.246 100.7) (width 0.5) (layer "B.Cu") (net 10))
 (segment (start 140.8 100.7) (end 143.25 100.7) (width 0.5) (layer "B.Cu") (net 10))
 (segment (start 155.023 98.459712) (end 155.023 99.477) (width 0.5) (layer "B.Cu") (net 10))
 (segment (start 143.7 100.25) (end 143.7 98.586712) (width 0.5) (layer "B.Cu") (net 10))
 (segment (start 143.25 100.7) (end 143.7 100.25) (width 0.5) (layer "B.Cu") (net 10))
 (segment (start 143.7 98.586712) (end 145.009712 97.277) (width 0.5) (layer "B.Cu") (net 10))
 (segment (start 153.840288 97.277) (end 155.023 98.459712) (width 0.5) (layer "B.Cu") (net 10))
 (segment (start 145.009712 97.277) (end 153.840288 97.277) (width 0.5) (layer "B.Cu") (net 10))
 (segment (start 143.886785 104.636785) (end 143.886785 106.150073) (width 0.5) (layer "B.Cu") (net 11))
 (segment (start 145.232712 107.496) (end 152.367288 107.496) (width 0.5) (layer "B.Cu") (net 11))
 (segment (start 143.7465 103.585134) (end 143.7465 104.4965) (width 0.5) (layer "B.Cu") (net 11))
 (segment (start 155.023 104.143842) (end 156.466842 102.7) (width 0.5) (layer "B.Cu") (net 11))
 (segment (start 141.3 102.7) (end 142.861366 102.7) (width 0.5) (layer "B.Cu") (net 11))
 (segment (start 142.861366 102.7) (end 143.7465 103.585134) (width 0.5) (layer "B.Cu") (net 11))
 (segment (start 143.7465 104.4965) (end 143.886785 104.636785) (width 0.5) (layer "B.Cu") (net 11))
 (segment (start 156.466842 102.7) (end 157.35 102.7) (width 0.5) (layer "B.Cu") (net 11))
 (segment (start 155.023 104.840288) (end 155.023 104.143842) (width 0.5) (layer "B.Cu") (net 11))
 (segment (start 143.886785 106.150073) (end 145.232712 107.496) (width 0.5) (layer "B.Cu") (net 11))
 (segment (start 152.367288 107.496) (end 155.023 104.840288) (width 0.5) (layer "B.Cu") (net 11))
 (segment (start 147.448 104.1375) (end 147.2355 104.35) (width 1) (layer "F.Cu") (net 13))
 (segment (start 149.198 101.077) (end 147.448 102.827) (width 1) (layer "F.Cu") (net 13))
 (segment (start 150.948 101.077) (end 149.198 101.077) (width 1) (layer "F.Cu") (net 13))
 (segment (start 147.448 102.827) (end 147.448 104.1375) (width 1) (layer "F.Cu") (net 13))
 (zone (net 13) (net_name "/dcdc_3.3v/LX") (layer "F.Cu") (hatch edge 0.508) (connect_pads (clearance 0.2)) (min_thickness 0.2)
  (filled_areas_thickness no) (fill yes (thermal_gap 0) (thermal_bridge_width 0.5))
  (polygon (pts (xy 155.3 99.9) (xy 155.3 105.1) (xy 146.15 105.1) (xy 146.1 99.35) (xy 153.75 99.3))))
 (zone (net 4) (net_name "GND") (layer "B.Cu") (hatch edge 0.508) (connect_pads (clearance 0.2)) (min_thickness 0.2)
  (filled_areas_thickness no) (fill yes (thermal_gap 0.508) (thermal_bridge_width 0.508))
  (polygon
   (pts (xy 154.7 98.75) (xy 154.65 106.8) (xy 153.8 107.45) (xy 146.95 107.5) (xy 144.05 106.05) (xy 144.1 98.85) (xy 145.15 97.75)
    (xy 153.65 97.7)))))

